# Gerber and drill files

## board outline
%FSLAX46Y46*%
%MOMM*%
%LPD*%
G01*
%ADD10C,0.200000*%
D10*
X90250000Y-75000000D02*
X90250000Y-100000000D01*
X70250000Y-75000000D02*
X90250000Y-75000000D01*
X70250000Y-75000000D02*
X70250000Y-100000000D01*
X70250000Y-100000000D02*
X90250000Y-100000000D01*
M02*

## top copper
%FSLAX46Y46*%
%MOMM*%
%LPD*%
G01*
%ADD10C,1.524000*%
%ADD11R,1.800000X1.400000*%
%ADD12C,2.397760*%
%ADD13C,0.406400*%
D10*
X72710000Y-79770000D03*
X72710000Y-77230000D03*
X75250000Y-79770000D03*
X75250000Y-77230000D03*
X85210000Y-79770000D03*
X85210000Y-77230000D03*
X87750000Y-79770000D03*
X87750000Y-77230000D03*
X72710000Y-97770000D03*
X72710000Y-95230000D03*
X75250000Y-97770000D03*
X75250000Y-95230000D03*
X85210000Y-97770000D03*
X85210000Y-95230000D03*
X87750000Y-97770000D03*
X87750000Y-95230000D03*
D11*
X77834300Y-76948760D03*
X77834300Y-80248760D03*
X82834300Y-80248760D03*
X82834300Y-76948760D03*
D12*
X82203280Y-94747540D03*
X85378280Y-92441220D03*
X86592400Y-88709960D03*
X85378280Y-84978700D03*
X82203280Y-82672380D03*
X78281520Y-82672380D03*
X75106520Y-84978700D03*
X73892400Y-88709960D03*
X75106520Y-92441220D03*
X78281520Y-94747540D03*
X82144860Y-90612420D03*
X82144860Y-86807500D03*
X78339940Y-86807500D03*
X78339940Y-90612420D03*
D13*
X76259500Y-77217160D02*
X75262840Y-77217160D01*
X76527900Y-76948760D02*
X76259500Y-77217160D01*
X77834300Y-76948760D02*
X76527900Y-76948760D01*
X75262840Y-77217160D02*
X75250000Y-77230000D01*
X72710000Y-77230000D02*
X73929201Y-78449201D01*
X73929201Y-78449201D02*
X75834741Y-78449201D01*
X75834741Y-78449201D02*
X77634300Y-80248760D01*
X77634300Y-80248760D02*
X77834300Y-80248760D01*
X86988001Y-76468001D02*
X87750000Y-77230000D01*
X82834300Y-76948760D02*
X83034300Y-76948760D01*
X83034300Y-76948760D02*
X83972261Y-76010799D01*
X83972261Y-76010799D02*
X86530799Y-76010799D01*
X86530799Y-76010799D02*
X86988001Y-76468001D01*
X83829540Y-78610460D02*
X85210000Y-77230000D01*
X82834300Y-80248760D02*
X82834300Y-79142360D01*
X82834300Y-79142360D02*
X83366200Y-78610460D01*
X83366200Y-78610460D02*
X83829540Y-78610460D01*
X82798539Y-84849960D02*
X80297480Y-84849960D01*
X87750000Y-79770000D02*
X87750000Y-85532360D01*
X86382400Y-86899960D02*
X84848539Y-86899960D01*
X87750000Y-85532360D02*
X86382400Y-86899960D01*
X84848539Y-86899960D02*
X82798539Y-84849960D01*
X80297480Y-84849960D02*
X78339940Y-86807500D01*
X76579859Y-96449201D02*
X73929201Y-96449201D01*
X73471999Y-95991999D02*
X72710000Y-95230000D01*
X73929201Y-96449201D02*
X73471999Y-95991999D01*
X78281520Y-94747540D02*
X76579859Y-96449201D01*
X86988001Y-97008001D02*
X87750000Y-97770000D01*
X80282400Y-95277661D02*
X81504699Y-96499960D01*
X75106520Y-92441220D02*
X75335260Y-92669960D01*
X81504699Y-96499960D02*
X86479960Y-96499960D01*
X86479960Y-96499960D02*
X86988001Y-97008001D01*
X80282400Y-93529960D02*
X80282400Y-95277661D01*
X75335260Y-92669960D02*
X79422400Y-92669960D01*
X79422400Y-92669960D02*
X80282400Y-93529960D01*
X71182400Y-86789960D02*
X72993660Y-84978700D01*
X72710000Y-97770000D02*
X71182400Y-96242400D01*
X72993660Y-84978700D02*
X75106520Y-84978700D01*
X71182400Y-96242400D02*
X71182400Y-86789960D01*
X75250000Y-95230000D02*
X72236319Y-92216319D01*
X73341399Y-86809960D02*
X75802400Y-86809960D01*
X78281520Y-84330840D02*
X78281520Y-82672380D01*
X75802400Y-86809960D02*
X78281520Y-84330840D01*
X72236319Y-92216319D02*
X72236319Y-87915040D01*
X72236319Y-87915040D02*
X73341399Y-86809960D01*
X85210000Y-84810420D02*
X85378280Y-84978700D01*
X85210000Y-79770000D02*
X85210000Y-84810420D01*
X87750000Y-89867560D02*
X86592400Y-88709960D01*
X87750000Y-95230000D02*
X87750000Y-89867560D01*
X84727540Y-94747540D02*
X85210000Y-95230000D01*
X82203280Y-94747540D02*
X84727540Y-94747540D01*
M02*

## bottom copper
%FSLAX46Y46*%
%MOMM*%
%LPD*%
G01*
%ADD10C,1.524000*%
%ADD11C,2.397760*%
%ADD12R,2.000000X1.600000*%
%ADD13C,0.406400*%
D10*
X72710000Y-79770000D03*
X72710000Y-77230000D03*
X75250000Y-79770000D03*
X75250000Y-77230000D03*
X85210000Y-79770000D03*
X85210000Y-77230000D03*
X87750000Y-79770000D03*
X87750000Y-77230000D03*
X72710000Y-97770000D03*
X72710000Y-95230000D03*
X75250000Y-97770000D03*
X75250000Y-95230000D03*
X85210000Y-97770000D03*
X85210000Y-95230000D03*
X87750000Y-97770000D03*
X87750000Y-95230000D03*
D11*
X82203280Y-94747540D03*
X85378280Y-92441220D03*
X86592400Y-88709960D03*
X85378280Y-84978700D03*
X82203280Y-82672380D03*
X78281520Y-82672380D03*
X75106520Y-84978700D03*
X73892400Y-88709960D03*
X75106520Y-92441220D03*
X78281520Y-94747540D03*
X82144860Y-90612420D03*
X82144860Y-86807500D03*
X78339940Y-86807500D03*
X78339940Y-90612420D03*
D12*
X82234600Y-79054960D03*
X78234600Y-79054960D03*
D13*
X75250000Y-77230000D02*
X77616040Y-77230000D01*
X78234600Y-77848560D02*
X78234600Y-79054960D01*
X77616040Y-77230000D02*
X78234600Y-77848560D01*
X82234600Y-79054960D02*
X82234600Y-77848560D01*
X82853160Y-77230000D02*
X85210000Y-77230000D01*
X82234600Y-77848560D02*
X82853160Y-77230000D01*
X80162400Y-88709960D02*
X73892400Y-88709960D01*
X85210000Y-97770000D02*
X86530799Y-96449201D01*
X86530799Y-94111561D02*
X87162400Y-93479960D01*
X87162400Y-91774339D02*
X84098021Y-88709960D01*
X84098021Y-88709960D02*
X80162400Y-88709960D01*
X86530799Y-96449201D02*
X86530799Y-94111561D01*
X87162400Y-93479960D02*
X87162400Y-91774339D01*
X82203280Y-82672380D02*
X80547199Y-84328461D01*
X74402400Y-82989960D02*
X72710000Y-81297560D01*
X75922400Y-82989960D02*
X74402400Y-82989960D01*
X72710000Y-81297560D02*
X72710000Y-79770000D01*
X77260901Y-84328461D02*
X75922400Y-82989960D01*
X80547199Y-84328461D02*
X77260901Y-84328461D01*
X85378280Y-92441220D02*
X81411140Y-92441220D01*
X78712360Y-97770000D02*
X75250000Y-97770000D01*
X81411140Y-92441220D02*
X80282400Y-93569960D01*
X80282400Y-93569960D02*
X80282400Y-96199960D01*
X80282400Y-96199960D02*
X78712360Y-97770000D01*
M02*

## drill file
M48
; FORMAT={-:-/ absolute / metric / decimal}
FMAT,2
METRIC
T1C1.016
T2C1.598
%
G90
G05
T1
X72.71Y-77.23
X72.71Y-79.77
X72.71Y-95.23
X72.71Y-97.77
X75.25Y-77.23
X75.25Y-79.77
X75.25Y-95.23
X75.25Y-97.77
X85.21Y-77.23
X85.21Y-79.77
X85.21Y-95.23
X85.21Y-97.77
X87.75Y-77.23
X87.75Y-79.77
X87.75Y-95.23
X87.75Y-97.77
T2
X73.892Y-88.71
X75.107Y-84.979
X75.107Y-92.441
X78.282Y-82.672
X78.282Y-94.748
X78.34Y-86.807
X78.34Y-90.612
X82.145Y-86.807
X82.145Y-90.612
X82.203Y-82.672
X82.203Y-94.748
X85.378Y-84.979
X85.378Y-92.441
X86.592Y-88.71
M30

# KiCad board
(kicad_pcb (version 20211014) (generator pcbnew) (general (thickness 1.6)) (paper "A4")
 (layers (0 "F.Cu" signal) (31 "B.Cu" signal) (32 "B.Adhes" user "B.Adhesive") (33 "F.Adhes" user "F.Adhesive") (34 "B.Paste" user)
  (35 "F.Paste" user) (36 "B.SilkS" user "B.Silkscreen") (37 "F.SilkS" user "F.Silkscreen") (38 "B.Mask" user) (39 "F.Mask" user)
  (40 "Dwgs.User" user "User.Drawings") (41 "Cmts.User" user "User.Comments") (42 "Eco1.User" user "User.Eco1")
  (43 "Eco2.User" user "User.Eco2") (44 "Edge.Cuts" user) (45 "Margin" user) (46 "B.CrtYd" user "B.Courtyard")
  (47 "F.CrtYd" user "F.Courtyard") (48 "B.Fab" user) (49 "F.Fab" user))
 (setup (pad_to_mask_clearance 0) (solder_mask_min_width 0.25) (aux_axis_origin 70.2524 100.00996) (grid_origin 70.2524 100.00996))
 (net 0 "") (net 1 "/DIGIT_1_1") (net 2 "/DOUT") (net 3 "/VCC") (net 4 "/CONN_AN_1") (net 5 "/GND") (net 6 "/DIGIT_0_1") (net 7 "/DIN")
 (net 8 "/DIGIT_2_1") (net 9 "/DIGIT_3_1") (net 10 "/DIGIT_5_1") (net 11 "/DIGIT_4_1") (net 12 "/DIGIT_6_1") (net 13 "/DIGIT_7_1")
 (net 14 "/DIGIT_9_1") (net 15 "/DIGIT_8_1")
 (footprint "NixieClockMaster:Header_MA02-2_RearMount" (layer "F.Cu") (at 75.25 78.5)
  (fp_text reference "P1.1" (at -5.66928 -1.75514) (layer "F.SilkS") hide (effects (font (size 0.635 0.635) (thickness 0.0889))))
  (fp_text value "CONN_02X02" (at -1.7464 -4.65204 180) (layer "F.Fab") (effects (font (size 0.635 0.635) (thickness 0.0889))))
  (pad "1" thru_hole circle (at -2.54 1.27) (size 1.524 1.524) (drill 1.016) (layers *.Cu *.Mask) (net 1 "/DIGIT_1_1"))
  (pad "2" thru_hole circle (at -2.54 -1.27) (size 1.524 1.524) (drill 1.016) (layers *.Cu *.Mask) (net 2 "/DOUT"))
  (pad "3" thru_hole circle (at 0 1.27) (size 1.524 1.524) (drill 1.016) (layers *.Cu *.Mask))
  (pad "4" thru_hole circle (at 0 -1.27) (size 1.524 1.524) (drill 1.016) (layers *.Cu *.Mask) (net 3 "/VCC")))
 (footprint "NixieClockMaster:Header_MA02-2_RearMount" (layer "F.Cu") (at 87.75 78.5)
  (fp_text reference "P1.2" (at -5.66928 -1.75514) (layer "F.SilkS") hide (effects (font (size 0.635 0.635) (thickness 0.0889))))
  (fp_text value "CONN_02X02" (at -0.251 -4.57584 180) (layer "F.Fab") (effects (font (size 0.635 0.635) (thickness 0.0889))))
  (pad "1" thru_hole circle (at -2.54 1.27) (size 1.524 1.524) (drill 1.016) (layers *.Cu *.Mask) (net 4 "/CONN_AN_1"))
  (pad "2" thru_hole circle (at -2.54 -1.27) (size 1.524 1.524) (drill 1.016) (layers *.Cu *.Mask) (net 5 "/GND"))
  (pad "3" thru_hole circle (at 0 1.27) (size 1.524 1.524) (drill 1.016) (layers *.Cu *.Mask) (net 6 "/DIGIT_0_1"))
  (pad "4" thru_hole circle (at 0 -1.27) (size 1.524 1.524) (drill 1.016) (layers *.Cu *.Mask) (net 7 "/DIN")))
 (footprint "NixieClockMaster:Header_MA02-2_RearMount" (layer "F.Cu") (at 75.25 96.5)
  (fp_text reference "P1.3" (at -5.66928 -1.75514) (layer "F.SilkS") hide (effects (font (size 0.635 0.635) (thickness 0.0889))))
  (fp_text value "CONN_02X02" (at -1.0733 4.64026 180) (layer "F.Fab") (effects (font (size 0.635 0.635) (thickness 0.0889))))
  (pad "1" thru_hole circle (at -2.54 1.27) (size 1.524 1.524) (drill 1.016) (layers *.Cu *.Mask) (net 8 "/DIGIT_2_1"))
  (pad "2" thru_hole circle (at -2.54 -1.27) (size 1.524 1.524) (drill 1.016) (layers *.Cu *.Mask) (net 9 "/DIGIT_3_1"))
  (pad "3" thru_hole circle (at 0 1.27) (size 1.524 1.524) (drill 1.016) (layers *.Cu *.Mask) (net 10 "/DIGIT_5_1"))
  (pad "4" thru_hole circle (at 0 -1.27) (size 1.524 1.524) (drill 1.016) (layers *.Cu *.Mask) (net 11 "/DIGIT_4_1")))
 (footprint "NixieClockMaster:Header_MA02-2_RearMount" (layer "F.Cu") (at 87.75 96.5)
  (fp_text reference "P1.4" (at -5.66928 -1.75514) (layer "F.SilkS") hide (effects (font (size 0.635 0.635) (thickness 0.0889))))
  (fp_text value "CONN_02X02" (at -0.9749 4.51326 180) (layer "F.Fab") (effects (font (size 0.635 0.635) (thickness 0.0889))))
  (pad "1" thru_hole circle (at -2.54 1.27) (size 1.524 1.524) (drill 1.016) (layers *.Cu *.Mask) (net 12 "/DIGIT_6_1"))
  (pad "2" thru_hole circle (at -2.54 -1.27) (size 1.524 1.524) (drill 1.016) (layers *.Cu *.Mask) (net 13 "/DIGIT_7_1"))
  (pad "3" thru_hole circle (at 0 1.27) (size 1.524 1.524) (drill 1.016) (layers *.Cu *.Mask) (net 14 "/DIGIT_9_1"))
  (pad "4" thru_hole circle (at 0 -1.27) (size 1.524 1.524) (drill 1.016) (layers *.Cu *.Mask) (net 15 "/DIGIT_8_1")))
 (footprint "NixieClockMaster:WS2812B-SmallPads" (layer "F.Cu") (at 80.3343 78.59876 90)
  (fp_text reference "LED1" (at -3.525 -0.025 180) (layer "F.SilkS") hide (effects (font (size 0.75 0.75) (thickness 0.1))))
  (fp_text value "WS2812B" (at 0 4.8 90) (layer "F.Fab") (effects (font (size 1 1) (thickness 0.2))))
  (pad "1" smd rect locked (at 1.65 -2.5 90) (size 1.4 1.8) (layers "F.Cu" "F.Paste" "F.Mask") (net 3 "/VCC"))
  (pad "2" smd rect locked (at -1.65 -2.5 90) (size 1.4 1.8) (layers "F.Cu" "F.Paste" "F.Mask") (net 2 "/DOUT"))
  (pad "3" smd rect locked (at -1.65 2.5 90) (size 1.4 1.8) (layers "F.Cu" "F.Paste" "F.Mask") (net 5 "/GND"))
  (pad "4" smd rect locked (at 1.65 2.5 90) (size 1.4 1.8) (layers "F.Cu" "F.Paste" "F.Mask") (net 7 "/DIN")))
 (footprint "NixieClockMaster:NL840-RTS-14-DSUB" (layer "F.Cu") (at 80.2424 88.70996 180)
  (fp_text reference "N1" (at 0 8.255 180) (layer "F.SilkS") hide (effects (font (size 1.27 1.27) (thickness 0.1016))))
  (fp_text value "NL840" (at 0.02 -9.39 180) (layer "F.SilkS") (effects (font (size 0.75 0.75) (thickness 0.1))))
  (pad "1" thru_hole circle (at -1.96088 -6.03758 180) (size 2.39776 2.39776) (drill 1.59766) (layers *.Cu *.Mask) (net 13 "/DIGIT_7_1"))
  (pad "2" thru_hole circle (at -5.13588 -3.73126 180) (size 2.39776 2.39776) (drill 1.59766) (layers *.Cu *.Mask) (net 10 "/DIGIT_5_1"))
  (pad "3" thru_hole circle (at -6.35 0 180) (size 2.39776 2.39776) (drill 1.59766) (layers *.Cu *.Mask) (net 15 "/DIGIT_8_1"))
  (pad "4" thru_hole circle (at -5.13588 3.73126 180) (size 2.39776 2.39776) (drill 1.59766) (layers *.Cu *.Mask) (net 4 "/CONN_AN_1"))
  (pad "5" thru_hole circle (at -1.96088 6.03758 180) (size 2.39776 2.39776) (drill 1.59766) (layers *.Cu *.Mask) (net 1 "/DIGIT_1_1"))
  (pad "6" thru_hole circle (at 1.96088 6.03758 180) (size 2.39776 2.39776) (drill 1.59766) (layers *.Cu *.Mask) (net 11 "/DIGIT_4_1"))
  (pad "7" thru_hole circle (at 5.13588 3.73126 180) (size 2.39776 2.39776) (drill 1.59766) (layers *.Cu *.Mask) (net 8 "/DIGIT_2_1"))
  (pad "8" thru_hole circle (at 6.35 0 180) (size 2.39776 2.39776) (drill 1.59766) (layers *.Cu *.Mask) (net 12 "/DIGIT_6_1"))
  (pad "9" thru_hole circle (at 5.13588 -3.73126 180) (size 2.39776 2.39776) (drill 1.59766) (layers *.Cu *.Mask) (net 14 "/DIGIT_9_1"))
  (pad "10" thru_hole circle (at 1.96088 -6.03758 180) (size 2.39776 2.39776) (drill 1.59766) (layers *.Cu *.Mask) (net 9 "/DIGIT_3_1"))
  (pad "11" thru_hole circle (at -1.90246 -1.90246 180) (size 2.39776 2.39776) (drill 1.59766) (layers *.Cu *.Mask))
  (pad "12" thru_hole circle (at -1.90246 1.90246 180) (size 2.39776 2.39776) (drill 1.59766) (layers *.Cu *.Mask))
  (pad "13" thru_hole circle (at 1.90246 1.90246 180) (size 2.39776 2.39776) (drill 1.59766) (layers *.Cu *.Mask) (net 6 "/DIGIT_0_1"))
  (pad "14" thru_hole circle (at 1.90246 -1.90246 180) (size 2.39776 2.39776) (drill 1.59766) (layers *.Cu *.Mask)))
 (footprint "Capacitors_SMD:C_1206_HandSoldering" (layer "B.Cu") (at 80.2346 79.05496 180)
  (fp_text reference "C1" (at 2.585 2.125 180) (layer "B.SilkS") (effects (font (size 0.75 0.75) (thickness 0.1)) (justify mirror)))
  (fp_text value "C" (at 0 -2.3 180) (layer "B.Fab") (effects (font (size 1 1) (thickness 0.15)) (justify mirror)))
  (pad "1" smd rect locked (at -2 0 180) (size 2 1.6) (layers "B.Cu" "B.Paste" "B.Mask") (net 5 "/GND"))
  (pad "2" smd rect locked (at 2 0 180) (size 2 1.6) (layers "B.Cu" "B.Paste" "B.Mask") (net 3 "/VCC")))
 (gr_line (start 90.25 75) (end 90.25 100) (layer "Edge.Cuts") (width 0.2))
 (gr_line (start 70.25 75) (end 90.25 75) (layer "Edge.Cuts") (width 0.2))
 (gr_line (start 70.25 75) (end 70.25 100) (layer "Edge.Cuts") (width 0.2))
 (gr_line (start 70.25 100) (end 90.25 100) (layer "Edge.Cuts") (width 0.2))
 (segment (start 76.2595 77.21716) (end 75.26284 77.21716) (width 0.4064) (layer "F.Cu") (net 3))
 (segment (start 76.5279 76.94876) (end 76.2595 77.21716) (width 0.4064) (layer "F.Cu") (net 3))
 (segment (start 77.8343 76.94876) (end 76.5279 76.94876) (width 0.4064) (layer "F.Cu") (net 3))
 (segment (start 75.26284 77.21716) (end 75.25 77.23) (width 0.4064) (layer "F.Cu") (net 3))
 (segment (start 75.25 77.23) (end 77.61604 77.23) (width 0.4064) (layer "B.Cu") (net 3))
 (segment (start 78.2346 77.84856) (end 78.2346 79.05496) (width 0.4064) (layer "B.Cu") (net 3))
 (segment (start 77.61604 77.23) (end 78.2346 77.84856) (width 0.4064) (layer "B.Cu") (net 3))
 (segment (start 72.71 77.23) (end 73.929201 78.449201) (width 0.4064) (layer "F.Cu") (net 2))
 (segment (start 73.929201 78.449201) (end 75.834741 78.449201) (width 0.4064) (layer "F.Cu") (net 2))
 (segment (start 75.834741 78.449201) (end 77.6343 80.24876) (width 0.4064) (layer "F.Cu") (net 2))
 (segment (start 77.6343 80.24876) (end 77.8343 80.24876) (width 0.4064) (layer "F.Cu") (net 2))
 (segment (start 86.988001 76.468001) (end 87.75 77.23) (width 0.4064) (layer "F.Cu") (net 7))
 (segment (start 82.8343 76.94876) (end 83.0343 76.94876) (width 0.4064) (layer "F.Cu") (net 7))
 (segment (start 83.0343 76.94876) (end 83.972261 76.010799) (width 0.4064) (layer "F.Cu") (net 7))
 (segment (start 83.972261 76.010799) (end 86.530799 76.010799) (width 0.4064) (layer "F.Cu") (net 7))
 (segment (start 86.530799 76.010799) (end 86.988001 76.468001) (width 0.4064) (layer "F.Cu") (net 7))
 (segment (start 83.82954 78.61046) (end 85.21 77.23) (width 0.4064) (layer "F.Cu") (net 5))
 (segment (start 82.8343 80.24876) (end 82.8343 79.14236) (width 0.4064) (layer "F.Cu") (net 5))
 (segment (start 82.8343 79.14236) (end 83.3662 78.61046) (width 0.4064) (layer "F.Cu") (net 5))
 (segment (start 83.3662 78.61046) (end 83.82954 78.61046) (width 0.4064) (layer "F.Cu") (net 5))
 (segment (start 82.2346 79.05496) (end 82.2346 77.84856) (width 0.4064) (layer "B.Cu") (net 5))
 (segment (start 82.85316 77.23) (end 85.21 77.23) (width 0.4064) (layer "B.Cu") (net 5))
 (segment (start 82.2346 77.84856) (end 82.85316 77.23) (width 0.4064) (layer "B.Cu") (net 5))
 (segment (start 82.798539 84.84996) (end 80.29748 84.84996) (width 0.4064) (layer "F.Cu") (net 6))
 (segment (start 87.75 79.77) (end 87.75 85.53236) (width 0.4064) (layer "F.Cu") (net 6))
 (segment (start 86.3824 86.89996) (end 84.848539 86.89996) (width 0.4064) (layer "F.Cu") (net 6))
 (segment (start 87.75 85.53236) (end 86.3824 86.89996) (width 0.4064) (layer "F.Cu") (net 6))
 (segment (start 84.848539 86.89996) (end 82.798539 84.84996) (width 0.4064) (layer "F.Cu") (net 6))
 (segment (start 80.29748 84.84996) (end 78.33994 86.8075) (width 0.4064) (layer "F.Cu") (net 6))
 (segment (start 76.579859 96.449201) (end 73.929201 96.449201) (width 0.4064) (layer "F.Cu") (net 9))
 (segment (start 73.471999 95.991999) (end 72.71 95.23) (width 0.4064) (layer "F.Cu") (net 9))
 (segment (start 73.929201 96.449201) (end 73.471999 95.991999) (width 0.4064) (layer "F.Cu") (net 9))
 (segment (start 78.28152 94.74754) (end 76.579859 96.449201) (width 0.4064) (layer "F.Cu") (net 9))
 (segment (start 86.988001 97.008001) (end 87.75 97.77) (width 0.4064) (layer "F.Cu") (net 14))
 (segment (start 80.2824 95.277661) (end 81.504699 96.49996) (width 0.4064) (layer "F.Cu") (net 14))
 (segment (start 75.10652 92.44122) (end 75.33526 92.66996) (width 0.4064) (layer "F.Cu") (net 14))
 (segment (start 81.504699 96.49996) (end 86.47996 96.49996) (width 0.4064) (layer "F.Cu") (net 14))
 (segment (start 86.47996 96.49996) (end 86.988001 97.008001) (width 0.4064) (layer "F.Cu") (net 14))
 (segment (start 80.2824 93.52996) (end 80.2824 95.277661) (width 0.4064) (layer "F.Cu") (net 14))
 (segment (start 75.33526 92.66996) (end 79.4224 92.66996) (width 0.4064) (layer "F.Cu") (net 14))
 (segment (start 79.4224 92.66996) (end 80.2824 93.52996) (width 0.4064) (layer "F.Cu") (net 14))
 (segment (start 80.1624 88.70996) (end 73.8924 88.70996) (width 0.4064) (layer "B.Cu") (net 12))
 (segment (start 85.21 97.77) (end 86.530799 96.449201) (width 0.4064) (layer "B.Cu") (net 12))
 (segment (start 86.530799 94.111561) (end 87.1624 93.47996) (width 0.4064) (layer "B.Cu") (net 12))
 (segment (start 87.1624 91.774339) (end 84.098021 88.70996) (width 0.4064) (layer "B.Cu") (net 12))
 (segment (start 84.098021 88.70996) (end 80.1624 88.70996) (width 0.4064) (layer "B.Cu") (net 12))
 (segment (start 86.530799 96.449201) (end 86.530799 94.111561) (width 0.4064) (layer "B.Cu") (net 12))
 (segment (start 87.1624 93.47996) (end 87.1624 91.774339) (width 0.4064) (layer "B.Cu") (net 12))
 (segment (start 71.1824 86.78996) (end 72.99366 84.9787) (width 0.4064) (layer "F.Cu") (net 8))
 (segment (start 72.71 97.77) (end 71.1824 96.2424) (width 0.4064) (layer "F.Cu") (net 8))
 (segment (start 72.99366 84.9787) (end 75.10652 84.9787) (width 0.4064) (layer "F.Cu") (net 8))
 (segment (start 71.1824 96.2424) (end 71.1824 86.78996) (width 0.4064) (layer "F.Cu") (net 8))
 (segment (start 75.25 95.23) (end 72.236319 92.216319) (width 0.4064) (layer "F.Cu") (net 11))
 (segment (start 73.341399 86.80996) (end 75.8024 86.80996) (width 0.4064) (layer "F.Cu") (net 11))
 (segment (start 78.28152 84.33084) (end 78.28152 82.67238) (width 0.4064) (layer "F.Cu") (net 11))
 (segment (start 75.8024 86.80996) (end 78.28152 84.33084) (width 0.4064) (layer "F.Cu") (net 11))
 (segment (start 72.236319 92.216319) (end 72.236319 87.91504) (width 0.4064) (layer "F.Cu") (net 11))
 (segment (start 72.236319 87.91504) (end 73.341399 86.80996) (width 0.4064) (layer "F.Cu") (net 11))
 (segment (start 82.20328 82.67238) (end 80.547199 84.328461) (width 0.4064) (layer "B.Cu") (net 1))
 (segment (start 74.4024 82.98996) (end 72.71 81.29756) (width 0.4064) (layer "B.Cu") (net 1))
 (segment (start 75.9224 82.98996) (end 74.4024 82.98996) (width 0.4064) (layer "B.Cu") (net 1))
 (segment (start 72.71 81.29756) (end 72.71 79.77) (width 0.4064) (layer "B.Cu") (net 1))
 (segment (start 77.260901 84.328461) (end 75.9224 82.98996) (width 0.4064) (layer "B.Cu") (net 1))
 (segment (start 80.547199 84.328461) (end 77.260901 84.328461) (width 0.4064) (layer "B.Cu") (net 1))
 (segment (start 85.21 84.81042) (end 85.37828 84.9787) (width 0.4064) (layer "F.Cu") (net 4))
 (segment (start 85.21 79.77) (end 85.21 84.81042) (width 0.4064) (layer "F.Cu") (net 4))
 (segment (start 87.75 89.86756) (end 86.5924 88.70996) (width 0.4064) (layer "F.Cu") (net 15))
 (segment (start 87.75 95.23) (end 87.75 89.86756) (width 0.4064) (layer "F.Cu") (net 15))
 (segment (start 85.37828 92.44122) (end 81.41114 92.44122) (width 0.4064) (layer "B.Cu") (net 10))
 (segment (start 78.71236 97.77) (end 75.25 97.77) (width 0.4064) (layer "B.Cu") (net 10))
 (segment (start 81.41114 92.44122) (end 80.2824 93.56996) (width 0.4064) (layer "B.Cu") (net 10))
 (segment (start 80.2824 93.56996) (end 80.2824 96.19996) (width 0.4064) (layer "B.Cu") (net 10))
 (segment (start 80.2824 96.19996) (end 78.71236 97.77) (width 0.4064) (layer "B.Cu") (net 10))
 (segment (start 84.72754 94.74754) (end 85.21 95.23) (width 0.4064) (layer "F.Cu") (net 13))
 (segment (start 82.20328 94.74754) (end 84.72754 94.74754) (width 0.4064) (layer "F.Cu") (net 13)))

